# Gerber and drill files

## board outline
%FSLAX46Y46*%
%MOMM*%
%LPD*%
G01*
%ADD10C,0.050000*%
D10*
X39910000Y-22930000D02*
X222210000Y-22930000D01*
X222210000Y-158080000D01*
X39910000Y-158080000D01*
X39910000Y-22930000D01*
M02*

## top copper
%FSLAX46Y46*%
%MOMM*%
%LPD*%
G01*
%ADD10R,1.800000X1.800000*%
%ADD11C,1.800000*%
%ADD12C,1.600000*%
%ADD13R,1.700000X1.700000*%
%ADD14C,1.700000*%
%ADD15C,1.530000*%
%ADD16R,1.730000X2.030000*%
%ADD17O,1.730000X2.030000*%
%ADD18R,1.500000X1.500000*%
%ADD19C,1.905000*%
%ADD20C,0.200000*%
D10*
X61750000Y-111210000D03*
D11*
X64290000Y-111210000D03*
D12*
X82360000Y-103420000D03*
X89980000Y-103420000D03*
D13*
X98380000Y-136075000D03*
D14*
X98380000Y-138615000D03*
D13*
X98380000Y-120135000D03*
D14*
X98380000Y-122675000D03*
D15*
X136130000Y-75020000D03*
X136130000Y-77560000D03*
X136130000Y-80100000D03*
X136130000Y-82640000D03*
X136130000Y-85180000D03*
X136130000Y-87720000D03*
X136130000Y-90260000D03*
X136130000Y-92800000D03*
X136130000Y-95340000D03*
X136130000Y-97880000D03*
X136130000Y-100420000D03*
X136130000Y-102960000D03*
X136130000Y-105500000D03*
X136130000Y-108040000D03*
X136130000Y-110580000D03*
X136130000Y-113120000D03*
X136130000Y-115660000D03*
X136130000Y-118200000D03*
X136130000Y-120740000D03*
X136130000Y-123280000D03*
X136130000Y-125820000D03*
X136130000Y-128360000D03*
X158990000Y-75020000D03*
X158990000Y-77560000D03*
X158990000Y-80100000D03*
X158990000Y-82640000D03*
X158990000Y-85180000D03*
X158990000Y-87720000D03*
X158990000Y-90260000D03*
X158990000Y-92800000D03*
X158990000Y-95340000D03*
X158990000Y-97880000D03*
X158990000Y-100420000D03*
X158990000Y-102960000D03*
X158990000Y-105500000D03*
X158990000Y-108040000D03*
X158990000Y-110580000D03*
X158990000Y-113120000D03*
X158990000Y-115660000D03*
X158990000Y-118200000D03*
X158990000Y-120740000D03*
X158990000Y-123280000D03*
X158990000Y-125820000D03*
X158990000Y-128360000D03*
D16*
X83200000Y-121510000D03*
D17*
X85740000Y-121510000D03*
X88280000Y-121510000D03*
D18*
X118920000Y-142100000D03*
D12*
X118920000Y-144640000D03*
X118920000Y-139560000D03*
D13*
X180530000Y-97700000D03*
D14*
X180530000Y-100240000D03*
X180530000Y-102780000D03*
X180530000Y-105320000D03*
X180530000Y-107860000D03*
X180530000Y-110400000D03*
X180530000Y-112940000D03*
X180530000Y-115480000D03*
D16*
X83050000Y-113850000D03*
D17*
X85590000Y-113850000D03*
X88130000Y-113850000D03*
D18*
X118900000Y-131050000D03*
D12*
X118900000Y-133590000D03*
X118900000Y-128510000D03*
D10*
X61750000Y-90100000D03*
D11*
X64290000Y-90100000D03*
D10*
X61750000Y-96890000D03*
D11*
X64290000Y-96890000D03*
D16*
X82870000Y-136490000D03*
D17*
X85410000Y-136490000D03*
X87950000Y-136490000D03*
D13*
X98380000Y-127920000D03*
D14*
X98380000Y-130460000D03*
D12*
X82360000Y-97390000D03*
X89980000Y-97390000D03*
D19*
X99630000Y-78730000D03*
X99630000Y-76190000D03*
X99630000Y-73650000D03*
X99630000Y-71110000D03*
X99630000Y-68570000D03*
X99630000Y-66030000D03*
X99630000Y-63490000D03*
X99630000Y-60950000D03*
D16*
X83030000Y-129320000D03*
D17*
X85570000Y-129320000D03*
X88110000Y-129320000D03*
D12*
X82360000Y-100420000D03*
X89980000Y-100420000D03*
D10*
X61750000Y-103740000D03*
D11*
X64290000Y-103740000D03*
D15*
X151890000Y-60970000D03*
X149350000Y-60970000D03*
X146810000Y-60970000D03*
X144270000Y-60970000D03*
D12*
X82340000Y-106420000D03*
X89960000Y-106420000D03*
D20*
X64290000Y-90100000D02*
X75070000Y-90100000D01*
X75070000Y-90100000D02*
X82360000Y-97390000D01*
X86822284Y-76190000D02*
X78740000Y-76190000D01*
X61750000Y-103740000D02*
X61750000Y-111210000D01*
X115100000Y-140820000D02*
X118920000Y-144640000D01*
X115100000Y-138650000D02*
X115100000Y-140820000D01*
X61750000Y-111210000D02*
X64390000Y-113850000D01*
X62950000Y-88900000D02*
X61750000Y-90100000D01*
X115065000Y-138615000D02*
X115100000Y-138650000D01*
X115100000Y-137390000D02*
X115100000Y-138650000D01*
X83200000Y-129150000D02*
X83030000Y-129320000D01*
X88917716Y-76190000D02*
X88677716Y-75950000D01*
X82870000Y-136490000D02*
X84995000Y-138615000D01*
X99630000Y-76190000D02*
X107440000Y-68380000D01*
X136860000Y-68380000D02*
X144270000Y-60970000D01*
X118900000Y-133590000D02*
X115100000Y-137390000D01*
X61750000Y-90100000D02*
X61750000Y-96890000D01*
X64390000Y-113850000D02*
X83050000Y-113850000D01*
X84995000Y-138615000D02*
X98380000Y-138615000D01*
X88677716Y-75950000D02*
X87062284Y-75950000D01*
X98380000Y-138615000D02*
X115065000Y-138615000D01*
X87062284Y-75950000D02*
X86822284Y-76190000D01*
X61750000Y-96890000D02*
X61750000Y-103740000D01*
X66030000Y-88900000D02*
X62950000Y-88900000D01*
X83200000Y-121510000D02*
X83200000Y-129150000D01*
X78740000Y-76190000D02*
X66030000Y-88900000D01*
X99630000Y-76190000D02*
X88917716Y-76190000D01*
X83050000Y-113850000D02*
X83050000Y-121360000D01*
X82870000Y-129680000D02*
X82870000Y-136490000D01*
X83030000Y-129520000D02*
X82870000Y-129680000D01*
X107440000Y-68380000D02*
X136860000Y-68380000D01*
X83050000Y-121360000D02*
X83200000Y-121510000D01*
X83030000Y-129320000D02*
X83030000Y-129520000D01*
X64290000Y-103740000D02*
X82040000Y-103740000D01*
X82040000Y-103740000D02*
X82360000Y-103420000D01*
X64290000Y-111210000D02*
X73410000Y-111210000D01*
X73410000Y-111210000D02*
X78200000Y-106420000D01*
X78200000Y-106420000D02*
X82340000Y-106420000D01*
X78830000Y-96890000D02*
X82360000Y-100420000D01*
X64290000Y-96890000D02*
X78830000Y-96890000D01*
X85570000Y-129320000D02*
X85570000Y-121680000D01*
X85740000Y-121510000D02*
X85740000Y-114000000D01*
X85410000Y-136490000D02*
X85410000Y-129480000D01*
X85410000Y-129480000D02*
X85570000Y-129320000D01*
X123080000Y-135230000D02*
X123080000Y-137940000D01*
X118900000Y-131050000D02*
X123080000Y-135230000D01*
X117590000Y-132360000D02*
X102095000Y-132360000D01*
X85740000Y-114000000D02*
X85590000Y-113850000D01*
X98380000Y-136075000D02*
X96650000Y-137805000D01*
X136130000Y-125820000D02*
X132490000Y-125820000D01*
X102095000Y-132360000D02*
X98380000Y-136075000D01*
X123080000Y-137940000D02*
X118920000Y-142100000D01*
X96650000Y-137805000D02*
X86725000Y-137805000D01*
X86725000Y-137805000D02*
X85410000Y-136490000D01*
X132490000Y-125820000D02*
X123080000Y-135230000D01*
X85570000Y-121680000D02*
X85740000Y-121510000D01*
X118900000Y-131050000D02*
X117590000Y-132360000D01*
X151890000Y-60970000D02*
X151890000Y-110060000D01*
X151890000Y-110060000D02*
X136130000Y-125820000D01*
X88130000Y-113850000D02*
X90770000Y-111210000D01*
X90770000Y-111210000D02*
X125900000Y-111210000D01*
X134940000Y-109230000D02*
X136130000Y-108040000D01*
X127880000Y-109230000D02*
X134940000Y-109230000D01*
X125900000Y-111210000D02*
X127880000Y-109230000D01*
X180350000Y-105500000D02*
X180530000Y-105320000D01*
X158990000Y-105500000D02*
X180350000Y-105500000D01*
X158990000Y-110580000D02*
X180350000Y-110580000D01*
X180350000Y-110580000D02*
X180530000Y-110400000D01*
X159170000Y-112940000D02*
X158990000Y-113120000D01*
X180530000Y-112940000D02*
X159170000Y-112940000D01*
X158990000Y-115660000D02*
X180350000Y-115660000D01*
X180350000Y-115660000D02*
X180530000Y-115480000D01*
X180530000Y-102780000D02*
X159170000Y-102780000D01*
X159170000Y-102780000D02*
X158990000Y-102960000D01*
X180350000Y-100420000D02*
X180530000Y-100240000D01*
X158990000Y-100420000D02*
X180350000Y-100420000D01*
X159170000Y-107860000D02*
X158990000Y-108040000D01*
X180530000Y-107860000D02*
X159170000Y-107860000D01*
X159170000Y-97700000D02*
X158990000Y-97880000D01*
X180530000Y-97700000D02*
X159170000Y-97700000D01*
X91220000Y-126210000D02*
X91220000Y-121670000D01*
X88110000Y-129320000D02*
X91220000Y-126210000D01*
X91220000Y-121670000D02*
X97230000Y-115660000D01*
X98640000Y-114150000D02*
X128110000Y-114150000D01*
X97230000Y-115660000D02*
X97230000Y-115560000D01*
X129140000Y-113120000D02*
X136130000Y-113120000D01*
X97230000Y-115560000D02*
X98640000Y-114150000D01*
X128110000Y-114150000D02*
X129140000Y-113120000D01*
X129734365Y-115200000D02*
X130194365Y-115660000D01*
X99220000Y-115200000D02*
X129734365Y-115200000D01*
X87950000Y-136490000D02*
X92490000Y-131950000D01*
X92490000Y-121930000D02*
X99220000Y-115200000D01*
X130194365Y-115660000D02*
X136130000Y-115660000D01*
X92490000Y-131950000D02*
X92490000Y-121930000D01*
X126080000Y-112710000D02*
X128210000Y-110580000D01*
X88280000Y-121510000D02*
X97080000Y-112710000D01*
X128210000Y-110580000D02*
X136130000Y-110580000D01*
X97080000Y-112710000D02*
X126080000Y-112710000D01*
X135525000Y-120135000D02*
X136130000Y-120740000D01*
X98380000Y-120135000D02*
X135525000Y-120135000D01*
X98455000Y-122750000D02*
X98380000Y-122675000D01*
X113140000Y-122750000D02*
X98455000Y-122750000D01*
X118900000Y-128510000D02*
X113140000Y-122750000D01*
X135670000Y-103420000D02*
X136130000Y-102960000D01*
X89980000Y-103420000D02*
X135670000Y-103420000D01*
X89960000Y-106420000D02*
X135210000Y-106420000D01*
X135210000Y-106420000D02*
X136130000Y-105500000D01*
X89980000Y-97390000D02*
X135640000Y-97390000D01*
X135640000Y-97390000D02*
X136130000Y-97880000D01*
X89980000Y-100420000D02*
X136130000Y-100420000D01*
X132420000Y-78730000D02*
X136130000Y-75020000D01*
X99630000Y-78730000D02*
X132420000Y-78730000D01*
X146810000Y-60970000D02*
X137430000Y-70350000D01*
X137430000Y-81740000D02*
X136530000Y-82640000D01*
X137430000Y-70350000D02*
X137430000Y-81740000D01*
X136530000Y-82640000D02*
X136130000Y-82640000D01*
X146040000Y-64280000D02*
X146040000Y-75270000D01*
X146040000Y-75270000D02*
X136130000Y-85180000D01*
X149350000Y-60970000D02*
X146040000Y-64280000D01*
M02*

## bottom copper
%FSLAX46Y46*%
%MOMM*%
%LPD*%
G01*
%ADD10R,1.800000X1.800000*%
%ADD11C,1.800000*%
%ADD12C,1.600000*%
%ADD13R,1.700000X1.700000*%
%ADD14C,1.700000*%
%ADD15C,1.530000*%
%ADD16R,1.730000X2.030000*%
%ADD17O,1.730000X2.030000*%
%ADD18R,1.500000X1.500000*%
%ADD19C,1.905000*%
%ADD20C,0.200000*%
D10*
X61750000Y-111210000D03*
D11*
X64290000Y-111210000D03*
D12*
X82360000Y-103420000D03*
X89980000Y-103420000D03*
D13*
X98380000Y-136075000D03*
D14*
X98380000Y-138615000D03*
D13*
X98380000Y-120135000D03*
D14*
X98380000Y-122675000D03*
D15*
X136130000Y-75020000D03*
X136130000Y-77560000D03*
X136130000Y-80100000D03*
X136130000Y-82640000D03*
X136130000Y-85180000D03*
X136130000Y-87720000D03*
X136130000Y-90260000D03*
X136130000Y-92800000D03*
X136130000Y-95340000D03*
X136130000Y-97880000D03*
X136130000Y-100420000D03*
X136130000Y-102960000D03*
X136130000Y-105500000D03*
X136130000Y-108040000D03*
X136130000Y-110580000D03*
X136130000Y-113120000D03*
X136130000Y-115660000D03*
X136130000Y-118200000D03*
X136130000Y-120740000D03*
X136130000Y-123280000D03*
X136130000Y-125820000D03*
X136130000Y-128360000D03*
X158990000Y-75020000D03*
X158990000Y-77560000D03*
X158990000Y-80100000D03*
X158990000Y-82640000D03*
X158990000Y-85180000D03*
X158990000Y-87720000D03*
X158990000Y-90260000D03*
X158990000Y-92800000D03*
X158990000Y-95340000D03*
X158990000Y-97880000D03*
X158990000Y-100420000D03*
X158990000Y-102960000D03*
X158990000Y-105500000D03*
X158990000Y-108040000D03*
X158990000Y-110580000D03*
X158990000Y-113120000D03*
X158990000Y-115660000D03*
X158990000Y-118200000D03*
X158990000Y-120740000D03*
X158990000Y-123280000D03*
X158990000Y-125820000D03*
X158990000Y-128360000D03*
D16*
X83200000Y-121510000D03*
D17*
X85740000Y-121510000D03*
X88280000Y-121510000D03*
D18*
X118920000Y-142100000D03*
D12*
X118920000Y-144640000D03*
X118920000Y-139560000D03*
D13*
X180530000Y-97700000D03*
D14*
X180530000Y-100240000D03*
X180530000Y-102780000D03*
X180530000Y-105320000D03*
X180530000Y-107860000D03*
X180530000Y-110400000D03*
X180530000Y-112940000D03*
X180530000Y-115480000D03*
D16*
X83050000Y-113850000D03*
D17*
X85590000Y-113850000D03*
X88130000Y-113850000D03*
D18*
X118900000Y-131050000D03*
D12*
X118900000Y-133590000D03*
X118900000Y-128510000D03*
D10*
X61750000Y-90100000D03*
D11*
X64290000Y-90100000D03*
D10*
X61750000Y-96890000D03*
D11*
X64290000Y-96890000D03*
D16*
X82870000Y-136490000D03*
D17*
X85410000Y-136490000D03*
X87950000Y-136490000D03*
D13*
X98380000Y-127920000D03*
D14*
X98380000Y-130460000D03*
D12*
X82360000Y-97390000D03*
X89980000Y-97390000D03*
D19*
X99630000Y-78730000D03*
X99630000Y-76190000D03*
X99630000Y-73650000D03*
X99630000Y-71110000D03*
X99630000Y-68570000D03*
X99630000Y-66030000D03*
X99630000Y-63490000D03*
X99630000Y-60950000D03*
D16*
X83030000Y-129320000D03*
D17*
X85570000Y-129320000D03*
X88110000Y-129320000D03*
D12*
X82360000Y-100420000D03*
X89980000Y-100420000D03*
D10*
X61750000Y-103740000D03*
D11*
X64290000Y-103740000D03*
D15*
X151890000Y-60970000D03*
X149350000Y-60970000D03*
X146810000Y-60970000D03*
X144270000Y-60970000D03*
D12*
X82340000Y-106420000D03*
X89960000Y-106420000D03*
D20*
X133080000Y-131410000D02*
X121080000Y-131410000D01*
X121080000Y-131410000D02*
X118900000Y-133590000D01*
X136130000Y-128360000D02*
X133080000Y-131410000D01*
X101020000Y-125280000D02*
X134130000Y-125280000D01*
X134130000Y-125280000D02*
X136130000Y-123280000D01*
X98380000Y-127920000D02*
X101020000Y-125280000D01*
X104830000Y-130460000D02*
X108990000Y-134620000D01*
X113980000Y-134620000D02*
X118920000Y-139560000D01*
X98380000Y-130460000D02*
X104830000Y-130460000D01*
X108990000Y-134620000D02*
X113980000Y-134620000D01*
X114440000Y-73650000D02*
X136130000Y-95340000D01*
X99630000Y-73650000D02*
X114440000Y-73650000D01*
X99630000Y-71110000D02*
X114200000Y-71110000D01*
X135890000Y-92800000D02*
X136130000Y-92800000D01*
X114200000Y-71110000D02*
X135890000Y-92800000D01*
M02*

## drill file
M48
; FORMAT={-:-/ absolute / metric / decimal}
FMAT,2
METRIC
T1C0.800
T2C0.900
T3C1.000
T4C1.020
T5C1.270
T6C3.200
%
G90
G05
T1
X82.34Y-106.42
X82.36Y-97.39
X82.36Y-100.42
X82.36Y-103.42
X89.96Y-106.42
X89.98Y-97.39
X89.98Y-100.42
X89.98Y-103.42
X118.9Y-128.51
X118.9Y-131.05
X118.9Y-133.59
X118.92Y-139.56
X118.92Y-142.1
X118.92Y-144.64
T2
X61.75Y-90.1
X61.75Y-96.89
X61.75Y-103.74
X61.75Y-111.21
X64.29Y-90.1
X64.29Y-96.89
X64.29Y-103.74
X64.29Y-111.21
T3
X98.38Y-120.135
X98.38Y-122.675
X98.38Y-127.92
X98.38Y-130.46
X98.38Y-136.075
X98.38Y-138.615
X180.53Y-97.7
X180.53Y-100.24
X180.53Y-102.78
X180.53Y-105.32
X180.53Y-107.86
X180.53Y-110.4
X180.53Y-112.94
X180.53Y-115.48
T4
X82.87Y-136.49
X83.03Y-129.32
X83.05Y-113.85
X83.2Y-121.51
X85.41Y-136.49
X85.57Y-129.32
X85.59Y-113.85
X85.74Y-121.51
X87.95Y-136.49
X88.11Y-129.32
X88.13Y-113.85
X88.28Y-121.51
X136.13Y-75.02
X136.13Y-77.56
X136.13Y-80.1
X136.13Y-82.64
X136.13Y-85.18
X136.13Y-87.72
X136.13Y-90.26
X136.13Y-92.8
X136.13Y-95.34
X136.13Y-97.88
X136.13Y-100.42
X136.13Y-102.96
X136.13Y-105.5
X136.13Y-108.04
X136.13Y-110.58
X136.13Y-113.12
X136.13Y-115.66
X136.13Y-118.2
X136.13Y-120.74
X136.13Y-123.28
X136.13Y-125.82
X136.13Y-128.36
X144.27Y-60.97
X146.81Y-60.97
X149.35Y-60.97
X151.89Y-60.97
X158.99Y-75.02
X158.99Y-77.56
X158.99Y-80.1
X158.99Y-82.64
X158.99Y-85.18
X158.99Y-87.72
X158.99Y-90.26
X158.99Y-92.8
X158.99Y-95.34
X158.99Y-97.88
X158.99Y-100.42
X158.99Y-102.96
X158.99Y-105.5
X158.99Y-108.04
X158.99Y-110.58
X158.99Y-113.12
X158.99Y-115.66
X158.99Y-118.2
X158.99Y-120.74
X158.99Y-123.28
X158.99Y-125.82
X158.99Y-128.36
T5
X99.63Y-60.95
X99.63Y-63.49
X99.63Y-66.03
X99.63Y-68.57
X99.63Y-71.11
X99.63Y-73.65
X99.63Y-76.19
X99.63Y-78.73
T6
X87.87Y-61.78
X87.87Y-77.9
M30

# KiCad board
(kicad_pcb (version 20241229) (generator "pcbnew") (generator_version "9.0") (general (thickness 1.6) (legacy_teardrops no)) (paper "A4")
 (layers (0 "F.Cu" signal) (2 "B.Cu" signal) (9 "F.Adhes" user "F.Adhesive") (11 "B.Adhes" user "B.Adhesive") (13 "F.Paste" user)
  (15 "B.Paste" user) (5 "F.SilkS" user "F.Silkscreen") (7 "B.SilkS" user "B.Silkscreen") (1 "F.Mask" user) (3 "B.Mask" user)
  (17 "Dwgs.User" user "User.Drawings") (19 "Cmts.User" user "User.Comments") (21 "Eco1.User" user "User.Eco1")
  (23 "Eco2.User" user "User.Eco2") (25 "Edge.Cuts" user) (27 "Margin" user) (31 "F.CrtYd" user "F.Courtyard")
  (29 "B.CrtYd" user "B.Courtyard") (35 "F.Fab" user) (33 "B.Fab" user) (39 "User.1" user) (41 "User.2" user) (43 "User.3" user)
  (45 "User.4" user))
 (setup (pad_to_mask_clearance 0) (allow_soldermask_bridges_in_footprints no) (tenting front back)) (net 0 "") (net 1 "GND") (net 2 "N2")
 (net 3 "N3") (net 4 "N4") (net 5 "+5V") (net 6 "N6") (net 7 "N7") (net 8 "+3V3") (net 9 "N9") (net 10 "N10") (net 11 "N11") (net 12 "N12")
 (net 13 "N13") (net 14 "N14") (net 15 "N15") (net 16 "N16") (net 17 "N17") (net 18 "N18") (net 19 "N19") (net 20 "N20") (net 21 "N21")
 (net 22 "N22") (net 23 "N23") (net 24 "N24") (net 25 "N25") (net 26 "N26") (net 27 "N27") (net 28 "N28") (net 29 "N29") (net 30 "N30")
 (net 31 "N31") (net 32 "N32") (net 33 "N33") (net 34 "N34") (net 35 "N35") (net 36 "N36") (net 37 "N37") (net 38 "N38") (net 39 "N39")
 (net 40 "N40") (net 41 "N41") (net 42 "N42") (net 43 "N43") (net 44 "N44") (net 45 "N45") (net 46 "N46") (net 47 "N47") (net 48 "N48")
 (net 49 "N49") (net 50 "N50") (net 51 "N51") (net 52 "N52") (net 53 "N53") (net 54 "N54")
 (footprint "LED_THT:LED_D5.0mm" (layer "F.Cu") (at 61.75 111.21)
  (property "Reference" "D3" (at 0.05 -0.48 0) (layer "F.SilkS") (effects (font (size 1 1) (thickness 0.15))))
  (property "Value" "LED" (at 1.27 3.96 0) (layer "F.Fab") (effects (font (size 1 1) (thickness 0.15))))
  (pad "1" thru_hole rect (at 0 0) (size 1.8 1.8) (drill 0.9) (layers "*.Cu" "*.Mask") (remove_unused_layers no) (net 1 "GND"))
  (pad "2" thru_hole circle (at 2.54 0) (size 1.8 1.8) (drill 0.9) (layers "*.Cu" "*.Mask") (remove_unused_layers no) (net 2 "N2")))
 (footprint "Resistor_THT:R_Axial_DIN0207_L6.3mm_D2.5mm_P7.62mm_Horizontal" (layer "F.Cu") (at 82.36 103.42)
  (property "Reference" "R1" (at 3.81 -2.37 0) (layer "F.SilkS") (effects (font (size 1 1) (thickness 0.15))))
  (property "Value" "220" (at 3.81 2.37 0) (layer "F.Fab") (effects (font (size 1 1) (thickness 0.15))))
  (pad "1" thru_hole circle (at 0 0) (size 1.6 1.6) (drill 0.8) (layers "*.Cu" "*.Mask") (remove_unused_layers no) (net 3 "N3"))
  (pad "2" thru_hole circle (at 7.62 0) (size 1.6 1.6) (drill 0.8) (layers "*.Cu" "*.Mask") (remove_unused_layers no) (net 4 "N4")))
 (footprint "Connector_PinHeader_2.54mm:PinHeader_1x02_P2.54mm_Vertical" (layer "F.Cu") (at 98.38 136.075)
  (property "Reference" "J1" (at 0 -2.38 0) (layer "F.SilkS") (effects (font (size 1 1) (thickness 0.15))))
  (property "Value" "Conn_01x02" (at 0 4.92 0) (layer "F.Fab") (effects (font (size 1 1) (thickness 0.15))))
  (pad "1" thru_hole rect (at 0 0) (size 1.7 1.7) (drill 1) (layers "*.Cu" "*.Mask") (remove_unused_layers no) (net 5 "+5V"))
  (pad "2" thru_hole circle (at 0 2.54) (size 1.7 1.7) (drill 1) (layers "*.Cu" "*.Mask") (remove_unused_layers no) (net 1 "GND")))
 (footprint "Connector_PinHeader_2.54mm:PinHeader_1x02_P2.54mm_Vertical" (layer "F.Cu") (at 98.38 120.135)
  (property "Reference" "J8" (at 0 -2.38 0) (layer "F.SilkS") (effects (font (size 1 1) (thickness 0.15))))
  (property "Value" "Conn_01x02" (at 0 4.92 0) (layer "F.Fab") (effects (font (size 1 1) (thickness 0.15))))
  (pad "1" thru_hole rect (at 0 0) (size 1.7 1.7) (drill 1) (layers "*.Cu" "*.Mask") (remove_unused_layers no) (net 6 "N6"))
  (pad "2" thru_hole circle (at 0 2.54) (size 1.7 1.7) (drill 1) (layers "*.Cu" "*.Mask") (remove_unused_layers no) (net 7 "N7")))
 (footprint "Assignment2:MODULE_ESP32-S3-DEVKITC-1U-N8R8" (layer "F.Cu") (at 147.56 104.99)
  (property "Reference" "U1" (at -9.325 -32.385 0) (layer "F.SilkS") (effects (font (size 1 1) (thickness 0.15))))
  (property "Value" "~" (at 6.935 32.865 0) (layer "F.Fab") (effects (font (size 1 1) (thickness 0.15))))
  (pad "J1_1" thru_hole circle (at -11.43 -29.97) (size 1.53 1.53) (drill 1.02) (layers "*.Cu" "*.Mask") (remove_unused_layers no)
   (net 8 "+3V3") (solder_mask_margin 0.102))
  (pad "J1_2" thru_hole circle (at -11.43 -27.43) (size 1.53 1.53) (drill 1.02) (layers "*.Cu" "*.Mask") (remove_unused_layers no)
   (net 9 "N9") (solder_mask_margin 0.102))
  (pad "J1_3" thru_hole circle (at -11.43 -24.89) (size 1.53 1.53) (drill 1.02) (layers "*.Cu" "*.Mask") (remove_unused_layers no)
   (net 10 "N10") (solder_mask_margin 0.102))
  (pad "J1_4" thru_hole circle (at -11.43 -22.35) (size 1.53 1.53) (drill 1.02) (layers "*.Cu" "*.Mask") (remove_unused_layers no)
   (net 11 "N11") (solder_mask_margin 0.102))
  (pad "J1_5" thru_hole circle (at -11.43 -19.81) (size 1.53 1.53) (drill 1.02) (layers "*.Cu" "*.Mask") (remove_unused_layers no)
   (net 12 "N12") (solder_mask_margin 0.102))
  (pad "J1_6" thru_hole circle (at -11.43 -17.27) (size 1.53 1.53) (drill 1.02) (layers "*.Cu" "*.Mask") (remove_unused_layers no)
   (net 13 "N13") (solder_mask_margin 0.102))
  (pad "J1_7" thru_hole circle (at -11.43 -14.73) (size 1.53 1.53) (drill 1.02) (layers "*.Cu" "*.Mask") (remove_unused_layers no)
   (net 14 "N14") (solder_mask_margin 0.102))
  (pad "J1_8" thru_hole circle (at -11.43 -12.19) (size 1.53 1.53) (drill 1.02) (layers "*.Cu" "*.Mask") (remove_unused_layers no)
   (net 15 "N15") (solder_mask_margin 0.102))
  (pad "J1_9" thru_hole circle (at -11.43 -9.65) (size 1.53 1.53) (drill 1.02) (layers "*.Cu" "*.Mask") (remove_unused_layers no)
   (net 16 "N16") (solder_mask_margin 0.102))
  (pad "J1_10" thru_hole circle (at -11.43 -7.11) (size 1.53 1.53) (drill 1.02) (layers "*.Cu" "*.Mask") (remove_unused_layers no)
   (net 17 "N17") (solder_mask_margin 0.102))
  (pad "J1_11" thru_hole circle (at -11.43 -4.57) (size 1.53 1.53) (drill 1.02) (layers "*.Cu" "*.Mask") (remove_unused_layers no)
   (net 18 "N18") (solder_mask_margin 0.102))
  (pad "J1_12" thru_hole circle (at -11.43 -2.03) (size 1.53 1.53) (drill 1.02) (layers "*.Cu" "*.Mask") (remove_unused_layers no)
   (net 4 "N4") (solder_mask_margin 0.102))
  (pad "J1_13" thru_hole circle (at -11.43 0.51) (size 1.53 1.53) (drill 1.02) (layers "*.Cu" "*.Mask") (remove_unused_layers no)
   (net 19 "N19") (solder_mask_margin 0.102))
  (pad "J1_14" thru_hole circle (at -11.43 3.05) (size 1.53 1.53) (drill 1.02) (layers "*.Cu" "*.Mask") (remove_unused_layers no)
   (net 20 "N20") (solder_mask_margin 0.102))
  (pad "J1_15" thru_hole circle (at -11.43 5.59) (size 1.53 1.53) (drill 1.02) (layers "*.Cu" "*.Mask") (remove_unused_layers no)
   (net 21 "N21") (solder_mask_margin 0.102))
  (pad "J1_16" thru_hole circle (at -11.43 8.13) (size 1.53 1.53) (drill 1.02) (layers "*.Cu" "*.Mask") (remove_unused_layers no)
   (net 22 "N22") (solder_mask_margin 0.102))
  (pad "J1_17" thru_hole circle (at -11.43 10.67) (size 1.53 1.53) (drill 1.02) (layers "*.Cu" "*.Mask") (remove_unused_layers no)
   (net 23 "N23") (solder_mask_margin 0.102))
  (pad "J1_18" thru_hole circle (at -11.43 13.21) (size 1.53 1.53) (drill 1.02) (layers "*.Cu" "*.Mask") (remove_unused_layers no)
   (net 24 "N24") (solder_mask_margin 0.102))
  (pad "J1_19" thru_hole circle (at -11.43 15.75) (size 1.53 1.53) (drill 1.02) (layers "*.Cu" "*.Mask") (remove_unused_layers no)
   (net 6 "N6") (solder_mask_margin 0.102))
  (pad "J1_20" thru_hole circle (at -11.43 18.29) (size 1.53 1.53) (drill 1.02) (layers "*.Cu" "*.Mask") (remove_unused_layers no)
   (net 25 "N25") (solder_mask_margin 0.102))
  (pad "J1_21" thru_hole circle (at -11.43 20.83) (size 1.53 1.53) (drill 1.02) (layers "*.Cu" "*.Mask") (remove_unused_layers no)
   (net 5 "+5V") (solder_mask_margin 0.102))
  (pad "J1_22" thru_hole circle (at -11.43 23.37) (size 1.53 1.53) (drill 1.02) (layers "*.Cu" "*.Mask") (remove_unused_layers no)
   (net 1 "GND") (solder_mask_margin 0.102))
  (pad "J3_1" thru_hole circle (at 11.43 -29.97) (size 1.53 1.53) (drill 1.02) (layers "*.Cu" "*.Mask") (remove_unused_layers no)
   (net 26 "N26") (solder_mask_margin 0.102))
  (pad "J3_2" thru_hole circle (at 11.43 -27.43) (size 1.53 1.53) (drill 1.02) (layers "*.Cu" "*.Mask") (remove_unused_layers no)
   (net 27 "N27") (solder_mask_margin 0.102))
  (pad "J3_3" thru_hole circle (at 11.43 -24.89) (size 1.53 1.53) (drill 1.02) (layers "*.Cu" "*.Mask") (remove_unused_layers no)
   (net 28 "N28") (solder_mask_margin 0.102))
  (pad "J3_4" thru_hole circle (at 11.43 -22.35) (size 1.53 1.53) (drill 1.02) (layers "*.Cu" "*.Mask") (remove_unused_layers no)
   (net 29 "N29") (solder_mask_margin 0.102))
  (pad "J3_5" thru_hole circle (at 11.43 -19.81) (size 1.53 1.53) (drill 1.02) (layers "*.Cu" "*.Mask") (remove_unused_layers no)
   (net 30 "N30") (solder_mask_margin 0.102))
  (pad "J3_6" thru_hole circle (at 11.43 -17.27) (size 1.53 1.53) (drill 1.02) (layers "*.Cu" "*.Mask") (remove_unused_layers no)
   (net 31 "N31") (solder_mask_margin 0.102))
  (pad "J3_7" thru_hole circle (at 11.43 -14.73) (size 1.53 1.53) (drill 1.02) (layers "*.Cu" "*.Mask") (remove_unused_layers no)
   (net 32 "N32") (solder_mask_margin 0.102))
  (pad "J3_8" thru_hole circle (at 11.43 -12.19) (size 1.53 1.53) (drill 1.02) (layers "*.Cu" "*.Mask") (remove_unused_layers no)
   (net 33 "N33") (solder_mask_margin 0.102))
  (pad "J3_9" thru_hole circle (at 11.43 -9.65) (size 1.53 1.53) (drill 1.02) (layers "*.Cu" "*.Mask") (remove_unused_layers no)
   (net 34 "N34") (solder_mask_margin 0.102))
  (pad "J3_10" thru_hole circle (at 11.43 -7.11) (size 1.53 1.53) (drill 1.02) (layers "*.Cu" "*.Mask") (remove_unused_layers no)
   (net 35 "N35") (solder_mask_margin 0.102))
  (pad "J3_11" thru_hole circle (at 11.43 -4.57) (size 1.53 1.53) (drill 1.02) (layers "*.Cu" "*.Mask") (remove_unused_layers no)
   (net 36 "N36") (solder_mask_margin 0.102))
  (pad "J3_12" thru_hole circle (at 11.43 -2.03) (size 1.53 1.53) (drill 1.02) (layers "*.Cu" "*.Mask") (remove_unused_layers no)
   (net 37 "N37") (solder_mask_margin 0.102))
  (pad "J3_13" thru_hole circle (at 11.43 0.51) (size 1.53 1.53) (drill 1.02) (layers "*.Cu" "*.Mask") (remove_unused_layers no)
   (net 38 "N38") (solder_mask_margin 0.102))
  (pad "J3_14" thru_hole circle (at 11.43 3.05) (size 1.53 1.53) (drill 1.02) (layers "*.Cu" "*.Mask") (remove_unused_layers no)
   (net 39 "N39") (solder_mask_margin 0.102))
  (pad "J3_15" thru_hole circle (at 11.43 5.59) (size 1.53 1.53) (drill 1.02) (layers "*.Cu" "*.Mask") (remove_unused_layers no)
   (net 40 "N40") (solder_mask_margin 0.102))
  (pad "J3_16" thru_hole circle (at 11.43 8.13) (size 1.53 1.53) (drill 1.02) (layers "*.Cu" "*.Mask") (remove_unused_layers no)
   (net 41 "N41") (solder_mask_margin 0.102))
  (pad "J3_17" thru_hole circle (at 11.43 10.67) (size 1.53 1.53) (drill 1.02) (layers "*.Cu" "*.Mask") (remove_unused_layers no)
   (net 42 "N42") (solder_mask_margin 0.102))
  (pad "J3_18" thru_hole circle (at 11.43 13.21) (size 1.53 1.53) (drill 1.02) (layers "*.Cu" "*.Mask") (remove_unused_layers no)
   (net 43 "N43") (solder_mask_margin 0.102))
  (pad "J3_19" thru_hole circle (at 11.43 15.75) (size 1.53 1.53) (drill 1.02) (layers "*.Cu" "*.Mask") (remove_unused_layers no)
   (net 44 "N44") (solder_mask_margin 0.102))
  (pad "J3_20" thru_hole circle (at 11.43 18.29) (size 1.53 1.53) (drill 1.02) (layers "*.Cu" "*.Mask") (remove_unused_layers no)
   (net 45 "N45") (solder_mask_margin 0.102))
  (pad "J3_21" thru_hole circle (at 11.43 20.83) (size 1.53 1.53) (drill 1.02) (layers "*.Cu" "*.Mask") (remove_unused_layers no)
   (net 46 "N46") (solder_mask_margin 0.102))
  (pad "J3_22" thru_hole circle (at 11.43 23.37) (size 1.53 1.53) (drill 1.02) (layers "*.Cu" "*.Mask") (remove_unused_layers no)
   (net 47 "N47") (solder_mask_margin 0.102)))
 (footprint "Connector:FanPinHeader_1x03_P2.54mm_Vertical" (layer "F.Cu") (at 83.2 121.51)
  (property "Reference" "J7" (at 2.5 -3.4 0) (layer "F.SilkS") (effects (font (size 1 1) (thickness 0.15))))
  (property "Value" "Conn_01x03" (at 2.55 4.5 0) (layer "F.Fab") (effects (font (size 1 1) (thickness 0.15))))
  (pad "1" thru_hole rect (at 0 0 90) (size 2.03 1.73) (drill 1.02) (layers "*.Cu" "*.Mask") (remove_unused_layers no) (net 1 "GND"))
  (pad "2" thru_hole oval (at 2.54 0 90) (size 2.03 1.73) (drill 1.02) (layers "*.Cu" "*.Mask") (remove_unused_layers no) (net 5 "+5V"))
  (pad "3" thru_hole oval (at 5.08 0 90) (size 2.03 1.73) (drill 1.02) (layers "*.Cu" "*.Mask") (remove_unused_layers no) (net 21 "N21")))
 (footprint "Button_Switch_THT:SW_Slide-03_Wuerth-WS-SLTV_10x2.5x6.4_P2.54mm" (layer "F.Cu") (at 118.92 142.1 90)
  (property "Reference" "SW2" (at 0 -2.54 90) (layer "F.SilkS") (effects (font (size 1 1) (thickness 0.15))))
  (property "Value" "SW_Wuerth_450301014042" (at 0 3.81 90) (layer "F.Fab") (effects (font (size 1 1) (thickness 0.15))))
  (pad "1" thru_hole rect (at 0 0 90) (size 1.5 1.5) (drill 0.8) (layers "*.Cu" "*.Mask") (remove_unused_layers no) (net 5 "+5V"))
  (pad "2" thru_hole circle (at -2.54 0 90) (size 1.6 1.6) (drill 0.8) (layers "*.Cu" "*.Mask") (remove_unused_layers no) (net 1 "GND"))
  (pad "3" thru_hole circle (at 2.54 0 90) (size 1.6 1.6) (drill 0.8) (layers "*.Cu" "*.Mask") (remove_unused_layers no) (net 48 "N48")))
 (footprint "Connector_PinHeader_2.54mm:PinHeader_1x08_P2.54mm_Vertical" (layer "F.Cu") (at 180.53 97.7)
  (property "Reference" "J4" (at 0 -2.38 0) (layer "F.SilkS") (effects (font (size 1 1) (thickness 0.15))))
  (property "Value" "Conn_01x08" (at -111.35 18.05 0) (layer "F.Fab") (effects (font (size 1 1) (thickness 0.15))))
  (pad "1" thru_hole rect (at 0 0) (size 1.7 1.7) (drill 1) (layers "*.Cu" "*.Mask") (remove_unused_layers no) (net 35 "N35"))
  (pad "2" thru_hole circle (at 0 2.54) (size 1.7 1.7) (drill 1) (layers "*.Cu" "*.Mask") (remove_unused_layers no) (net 36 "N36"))
  (pad "3" thru_hole circle (at 0 5.08) (size 1.7 1.7) (drill 1) (layers "*.Cu" "*.Mask") (remove_unused_layers no) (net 37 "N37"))
  (pad "4" thru_hole circle (at 0 7.62) (size 1.7 1.7) (drill 1) (layers "*.Cu" "*.Mask") (remove_unused_layers no) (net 38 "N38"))
  (pad "5" thru_hole circle (at 0 10.16) (size 1.7 1.7) (drill 1) (layers "*.Cu" "*.Mask") (remove_unused_layers no) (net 39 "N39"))
  (pad "6" thru_hole circle (at 0 12.7) (size 1.7 1.7) (drill 1) (layers "*.Cu" "*.Mask") (remove_unused_layers no) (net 40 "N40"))
  (pad "7" thru_hole circle (at 0 15.24) (size 1.7 1.7) (drill 1) (layers "*.Cu" "*.Mask") (remove_unused_layers no) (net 41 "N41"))
  (pad "8" thru_hole circle (at 0 17.78) (size 1.7 1.7) (drill 1) (layers "*.Cu" "*.Mask") (remove_unused_layers no) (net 42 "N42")))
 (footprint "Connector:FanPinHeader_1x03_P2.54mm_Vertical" (layer "F.Cu") (at 83.05 113.85)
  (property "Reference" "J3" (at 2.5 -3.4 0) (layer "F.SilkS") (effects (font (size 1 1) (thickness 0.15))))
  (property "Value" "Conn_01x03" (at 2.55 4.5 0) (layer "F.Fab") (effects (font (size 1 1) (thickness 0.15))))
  (pad "1" thru_hole rect (at 0 0 90) (size 2.03 1.73) (drill 1.02) (layers "*.Cu" "*.Mask") (remove_unused_layers no) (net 1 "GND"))
  (pad "2" thru_hole oval (at 2.54 0 90) (size 2.03 1.73) (drill 1.02) (layers "*.Cu" "*.Mask") (remove_unused_layers no) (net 5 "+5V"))
  (pad "3" thru_hole oval (at 5.08 0 90) (size 2.03 1.73) (drill 1.02) (layers "*.Cu" "*.Mask") (remove_unused_layers no) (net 20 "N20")))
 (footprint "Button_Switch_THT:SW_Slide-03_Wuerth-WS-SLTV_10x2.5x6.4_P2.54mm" (layer "F.Cu") (at 118.9 131.05 90)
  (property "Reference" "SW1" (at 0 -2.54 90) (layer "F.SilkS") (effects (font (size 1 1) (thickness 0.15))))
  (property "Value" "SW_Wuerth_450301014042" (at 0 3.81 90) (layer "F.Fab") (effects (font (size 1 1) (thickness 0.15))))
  (pad "1" thru_hole rect (at 0 0 90) (size 1.5 1.5) (drill 0.8) (layers "*.Cu" "*.Mask") (remove_unused_layers no) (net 5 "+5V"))
  (pad "2" thru_hole circle (at -2.54 0 90) (size 1.6 1.6) (drill 0.8) (layers "*.Cu" "*.Mask") (remove_unused_layers no) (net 1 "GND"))
  (pad "3" thru_hole circle (at 2.54 0 90) (size 1.6 1.6) (drill 0.8) (layers "*.Cu" "*.Mask") (remove_unused_layers no) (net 7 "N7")))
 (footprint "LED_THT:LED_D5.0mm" (layer "F.Cu") (at 61.75 90.1)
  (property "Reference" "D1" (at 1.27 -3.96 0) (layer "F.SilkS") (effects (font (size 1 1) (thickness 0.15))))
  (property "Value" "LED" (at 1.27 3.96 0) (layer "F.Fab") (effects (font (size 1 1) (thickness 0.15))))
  (pad "1" thru_hole rect (at 0 0) (size 1.8 1.8) (drill 0.9) (layers "*.Cu" "*.Mask") (remove_unused_layers no) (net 1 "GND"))
  (pad "2" thru_hole circle (at 2.54 0) (size 1.8 1.8) (drill 0.9) (layers "*.Cu" "*.Mask") (remove_unused_layers no) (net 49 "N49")))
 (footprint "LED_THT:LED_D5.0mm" (layer "F.Cu") (at 61.75 96.89)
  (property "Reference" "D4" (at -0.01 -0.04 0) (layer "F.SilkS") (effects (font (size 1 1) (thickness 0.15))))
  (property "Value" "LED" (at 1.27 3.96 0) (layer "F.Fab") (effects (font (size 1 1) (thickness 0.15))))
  (pad "1" thru_hole rect (at 0 0) (size 1.8 1.8) (drill 0.9) (layers "*.Cu" "*.Mask") (remove_unused_layers no) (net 1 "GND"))
  (pad "2" thru_hole circle (at 2.54 0) (size 1.8 1.8) (drill 0.9) (layers "*.Cu" "*.Mask") (remove_unused_layers no) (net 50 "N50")))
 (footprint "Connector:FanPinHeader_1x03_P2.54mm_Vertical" (layer "F.Cu") (at 82.87 136.49)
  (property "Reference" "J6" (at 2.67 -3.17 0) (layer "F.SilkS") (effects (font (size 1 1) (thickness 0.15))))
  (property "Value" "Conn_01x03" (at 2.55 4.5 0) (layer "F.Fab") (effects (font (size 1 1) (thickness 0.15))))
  (pad "1" thru_hole rect (at 0 0 90) (size 2.03 1.73) (drill 1.02) (layers "*.Cu" "*.Mask") (remove_unused_layers no) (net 1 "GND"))
  (pad "2" thru_hole oval (at 2.54 0 90) (size 2.03 1.73) (drill 1.02) (layers "*.Cu" "*.Mask") (remove_unused_layers no) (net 5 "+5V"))
  (pad "3" thru_hole oval (at 5.08 0 90) (size 2.03 1.73) (drill 1.02) (layers "*.Cu" "*.Mask") (remove_unused_layers no) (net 23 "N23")))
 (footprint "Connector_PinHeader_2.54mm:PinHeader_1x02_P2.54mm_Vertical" (layer "F.Cu") (at 98.38 127.92)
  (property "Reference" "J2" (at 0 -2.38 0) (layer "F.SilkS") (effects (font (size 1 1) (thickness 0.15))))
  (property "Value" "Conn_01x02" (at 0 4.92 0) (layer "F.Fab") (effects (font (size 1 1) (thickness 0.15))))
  (pad "1" thru_hole rect (at 0 0) (size 1.7 1.7) (drill 1) (layers "*.Cu" "*.Mask") (remove_unused_layers no) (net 25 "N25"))
  (pad "2" thru_hole circle (at 0 2.54) (size 1.7 1.7) (drill 1) (layers "*.Cu" "*.Mask") (remove_unused_layers no) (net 48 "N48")))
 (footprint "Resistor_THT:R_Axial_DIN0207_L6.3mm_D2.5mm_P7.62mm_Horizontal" (layer "F.Cu") (at 82.36 97.39)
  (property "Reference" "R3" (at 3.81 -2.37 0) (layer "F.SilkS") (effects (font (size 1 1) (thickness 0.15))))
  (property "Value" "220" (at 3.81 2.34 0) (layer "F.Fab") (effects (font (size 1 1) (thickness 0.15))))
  (pad "1" thru_hole circle (at 0 0) (size 1.6 1.6) (drill 0.8) (layers "*.Cu" "*.Mask") (remove_unused_layers no) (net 49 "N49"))
  (pad "2" thru_hole circle (at 7.62 0) (size 1.6 1.6) (drill 0.8) (layers "*.Cu" "*.Mask") (remove_unused_layers no) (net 17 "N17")))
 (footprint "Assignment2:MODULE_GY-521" (layer "F.Cu") (at 93.3 69.84 180)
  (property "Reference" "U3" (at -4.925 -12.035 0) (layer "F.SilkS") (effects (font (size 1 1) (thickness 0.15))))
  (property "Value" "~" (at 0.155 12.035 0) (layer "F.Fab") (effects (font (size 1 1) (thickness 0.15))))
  (pad "" np_thru_hole circle (at 5.43 -8.06 180) (size 3.2 3.2) (drill 3.2) (layers "*.Cu" "*.Mask"))
  (pad "" np_thru_hole circle (at 5.43 8.06 180) (size 3.2 3.2) (drill 3.2) (layers "*.Cu" "*.Mask"))
  (pad "1" thru_hole circle (at -6.33 -8.89 180) (size 1.905 1.905) (drill 1.27) (layers "*.Cu" "*.Mask") (remove_unused_layers no)
   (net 8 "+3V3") (solder_mask_margin 0.102))
  (pad "2" thru_hole circle (at -6.33 -6.35 180) (size 1.905 1.905) (drill 1.27) (layers "*.Cu" "*.Mask") (remove_unused_layers no)
   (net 1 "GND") (solder_mask_margin 0.102))
  (pad "3" thru_hole circle (at -6.33 -3.81 180) (size 1.905 1.905) (drill 1.27) (layers "*.Cu" "*.Mask") (remove_unused_layers no)
   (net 16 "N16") (solder_mask_margin 0.102))
  (pad "4" thru_hole circle (at -6.33 -1.27 180) (size 1.905 1.905) (drill 1.27) (layers "*.Cu" "*.Mask") (remove_unused_layers no)
   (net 15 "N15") (solder_mask_margin 0.102))
  (pad "5" thru_hole circle (at -6.33 1.27 180) (size 1.905 1.905) (drill 1.27) (layers "*.Cu" "*.Mask") (remove_unused_layers no)
   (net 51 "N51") (solder_mask_margin 0.102))
  (pad "6" thru_hole circle (at -6.33 3.81 180) (size 1.905 1.905) (drill 1.27) (layers "*.Cu" "*.Mask") (remove_unused_layers no)
   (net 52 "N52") (solder_mask_margin 0.102))
  (pad "7" thru_hole circle (at -6.33 6.35 180) (size 1.905 1.905) (drill 1.27) (layers "*.Cu" "*.Mask") (remove_unused_layers no)
   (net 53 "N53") (solder_mask_margin 0.102))
  (pad "8" thru_hole circle (at -6.33 8.89 180) (size 1.905 1.905) (drill 1.27) (layers "*.Cu" "*.Mask") (remove_unused_layers no)
   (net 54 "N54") (solder_mask_margin 0.102)))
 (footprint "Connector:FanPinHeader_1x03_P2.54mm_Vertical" (layer "F.Cu") (at 83.03 129.32)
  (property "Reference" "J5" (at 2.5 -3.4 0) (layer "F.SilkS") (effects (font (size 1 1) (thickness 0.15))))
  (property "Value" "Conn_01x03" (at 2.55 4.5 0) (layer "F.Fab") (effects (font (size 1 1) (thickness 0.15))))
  (pad "1" thru_hole rect (at 0 0 90) (size 2.03 1.73) (drill 1.02) (layers "*.Cu" "*.Mask") (remove_unused_layers no) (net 1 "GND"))
  (pad "2" thru_hole oval (at 2.54 0 90) (size 2.03 1.73) (drill 1.02) (layers "*.Cu" "*.Mask") (remove_unused_layers no) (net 5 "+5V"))
  (pad "3" thru_hole oval (at 5.08 0 90) (size 2.03 1.73) (drill 1.02) (layers "*.Cu" "*.Mask") (remove_unused_layers no) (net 22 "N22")))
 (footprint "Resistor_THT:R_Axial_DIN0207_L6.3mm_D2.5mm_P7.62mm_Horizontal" (layer "F.Cu") (at 82.36 100.42)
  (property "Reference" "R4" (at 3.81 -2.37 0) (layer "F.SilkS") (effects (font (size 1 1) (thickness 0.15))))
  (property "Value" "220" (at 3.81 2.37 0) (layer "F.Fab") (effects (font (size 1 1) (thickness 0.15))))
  (pad "1" thru_hole circle (at 0 0) (size 1.6 1.6) (drill 0.8) (layers "*.Cu" "*.Mask") (remove_unused_layers no) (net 50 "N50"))
  (pad "2" thru_hole circle (at 7.62 0) (size 1.6 1.6) (drill 0.8) (layers "*.Cu" "*.Mask") (remove_unused_layers no) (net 18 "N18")))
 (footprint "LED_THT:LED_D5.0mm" (layer "F.Cu") (at 61.75 103.74)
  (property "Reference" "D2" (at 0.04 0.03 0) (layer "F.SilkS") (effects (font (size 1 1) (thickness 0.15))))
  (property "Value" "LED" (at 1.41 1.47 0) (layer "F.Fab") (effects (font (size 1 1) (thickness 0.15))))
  (pad "1" thru_hole rect (at 0 0) (size 1.8 1.8) (drill 0.9) (layers "*.Cu" "*.Mask") (remove_unused_layers no) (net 1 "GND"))
  (pad "2" thru_hole circle (at 2.54 0) (size 1.8 1.8) (drill 0.9) (layers "*.Cu" "*.Mask") (remove_unused_layers no) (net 3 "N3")))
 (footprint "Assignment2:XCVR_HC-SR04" (layer "F.Cu") (at 148.08 60.97 180)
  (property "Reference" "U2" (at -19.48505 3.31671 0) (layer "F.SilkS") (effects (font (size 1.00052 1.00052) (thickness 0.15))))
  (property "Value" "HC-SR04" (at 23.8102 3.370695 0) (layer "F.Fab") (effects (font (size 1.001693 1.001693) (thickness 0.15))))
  (pad "1" thru_hole circle (at -3.81 0 180) (size 1.53 1.53) (drill 1.02) (layers "*.Cu" "*.Mask") (remove_unused_layers no) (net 5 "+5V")
   (solder_mask_margin 0.102))
  (pad "2" thru_hole circle (at -1.27 0 180) (size 1.53 1.53) (drill 1.02) (layers "*.Cu" "*.Mask") (remove_unused_layers no) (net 12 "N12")
   (solder_mask_margin 0.102))
  (pad "3" thru_hole circle (at 1.27 0 180) (size 1.53 1.53) (drill 1.02) (layers "*.Cu" "*.Mask") (remove_unused_layers no) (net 11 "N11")
   (solder_mask_margin 0.102))
  (pad "4" thru_hole circle (at 3.81 0 180) (size 1.53 1.53) (drill 1.02) (layers "*.Cu" "*.Mask") (remove_unused_layers no) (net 1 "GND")
   (solder_mask_margin 0.102)))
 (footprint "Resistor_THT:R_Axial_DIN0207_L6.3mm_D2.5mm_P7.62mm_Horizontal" (layer "F.Cu") (at 82.34 106.42)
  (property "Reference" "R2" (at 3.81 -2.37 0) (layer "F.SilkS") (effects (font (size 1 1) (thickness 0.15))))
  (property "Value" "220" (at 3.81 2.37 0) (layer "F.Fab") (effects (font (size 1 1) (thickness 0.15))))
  (pad "1" thru_hole circle (at 0 0) (size 1.6 1.6) (drill 0.8) (layers "*.Cu" "*.Mask") (remove_unused_layers no) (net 2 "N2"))
  (pad "2" thru_hole circle (at 7.62 0) (size 1.6 1.6) (drill 0.8) (layers "*.Cu" "*.Mask") (remove_unused_layers no) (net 19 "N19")))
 (gr_rect (start 39.91 22.93) (end 222.21 158.08) (stroke (width 0.05) (type default)) (fill no) (layer "Edge.Cuts"))
 (segment (start 64.29 90.1) (end 75.07 90.1) (width 0.2) (layer "F.Cu") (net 49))
 (segment (start 75.07 90.1) (end 82.36 97.39) (width 0.2) (layer "F.Cu") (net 49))
 (segment (start 86.822284 76.19) (end 78.74 76.19) (width 0.2) (layer "F.Cu") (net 1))
 (segment (start 61.75 103.74) (end 61.75 111.21) (width 0.2) (layer "F.Cu") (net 1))
 (segment (start 115.1 140.82) (end 118.92 144.64) (width 0.2) (layer "F.Cu") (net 1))
 (segment (start 115.1 138.65) (end 115.1 140.82) (width 0.2) (layer "F.Cu") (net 1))
 (segment (start 61.75 111.21) (end 64.39 113.85) (width 0.2) (layer "F.Cu") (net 1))
 (segment (start 62.95 88.9) (end 61.75 90.1) (width 0.2) (layer "F.Cu") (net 1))
 (segment (start 115.065 138.615) (end 115.1 138.65) (width 0.2) (layer "F.Cu") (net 1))
 (segment (start 115.1 137.39) (end 115.1 138.65) (width 0.2) (layer "F.Cu") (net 1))
 (segment (start 83.2 129.15) (end 83.03 129.32) (width 0.2) (layer "F.Cu") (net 1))
 (segment (start 88.917716 76.19) (end 88.677716 75.95) (width 0.2) (layer "F.Cu") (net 1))
 (segment (start 82.87 136.49) (end 84.995 138.615) (width 0.2) (layer "F.Cu") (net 1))
 (segment (start 99.63 76.19) (end 107.44 68.38) (width 0.2) (layer "F.Cu") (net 1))
 (segment (start 136.86 68.38) (end 144.27 60.97) (width 0.2) (layer "F.Cu") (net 1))
 (segment (start 118.9 133.59) (end 115.1 137.39) (width 0.2) (layer "F.Cu") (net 1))
 (segment (start 61.75 90.1) (end 61.75 96.89) (width 0.2) (layer "F.Cu") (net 1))
 (segment (start 64.39 113.85) (end 83.05 113.85) (width 0.2) (layer "F.Cu") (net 1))
 (segment (start 84.995 138.615) (end 98.38 138.615) (width 0.2) (layer "F.Cu") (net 1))
 (segment (start 88.677716 75.95) (end 87.062284 75.95) (width 0.2) (layer "F.Cu") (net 1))
 (segment (start 98.38 138.615) (end 115.065 138.615) (width 0.2) (layer "F.Cu") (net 1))
 (segment (start 87.062284 75.95) (end 86.822284 76.19) (width 0.2) (layer "F.Cu") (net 1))
 (segment (start 61.75 96.89) (end 61.75 103.74) (width 0.2) (layer "F.Cu") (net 1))
 (segment (start 66.03 88.9) (end 62.95 88.9) (width 0.2) (layer "F.Cu") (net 1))
 (segment (start 83.2 121.51) (end 83.2 129.15) (width 0.2) (layer "F.Cu") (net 1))
 (segment (start 78.74 76.19) (end 66.03 88.9) (width 0.2) (layer "F.Cu") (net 1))
 (segment (start 99.63 76.19) (end 88.917716 76.19) (width 0.2) (layer "F.Cu") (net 1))
 (segment (start 83.05 113.85) (end 83.05 121.36) (width 0.2) (layer "F.Cu") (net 1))
 (segment (start 82.87 129.68) (end 82.87 136.49) (width 0.2) (layer "F.Cu") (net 1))
 (segment (start 83.03 129.52) (end 82.87 129.68) (width 0.2) (layer "F.Cu") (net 1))
 (segment (start 107.44 68.38) (end 136.86 68.38) (width 0.2) (layer "F.Cu") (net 1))
 (segment (start 83.05 121.36) (end 83.2 121.51) (width 0.2) (layer "F.Cu") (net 1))
 (segment (start 83.03 129.32) (end 83.03 129.52) (width 0.2) (layer "F.Cu") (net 1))
 (segment (start 133.08 131.41) (end 121.08 131.41) (width 0.2) (layer "B.Cu") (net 1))
 (segment (start 121.08 131.41) (end 118.9 133.59) (width 0.2) (layer "B.Cu") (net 1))
 (segment (start 136.13 128.36) (end 133.08 131.41) (width 0.2) (layer "B.Cu") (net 1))
 (segment (start 64.29 103.74) (end 82.04 103.74) (width 0.2) (layer "F.Cu") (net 3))
 (segment (start 82.04 103.74) (end 82.36 103.42) (width 0.2) (layer "F.Cu") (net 3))
 (segment (start 64.29 111.21) (end 73.41 111.21) (width 0.2) (layer "F.Cu") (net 2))
 (segment (start 73.41 111.21) (end 78.2 106.42) (width 0.2) (layer "F.Cu") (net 2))
 (segment (start 78.2 106.42) (end 82.34 106.42) (width 0.2) (layer "F.Cu") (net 2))
 (segment (start 78.83 96.89) (end 82.36 100.42) (width 0.2) (layer "F.Cu") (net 50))
 (segment (start 64.29 96.89) (end 78.83 96.89) (width 0.2) (layer "F.Cu") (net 50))
 (segment (start 85.57 129.32) (end 85.57 121.68) (width 0.2) (layer "F.Cu") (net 5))
 (segment (start 85.74 121.51) (end 85.74 114) (width 0.2) (layer "F.Cu") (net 5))
 (segment (start 85.41 136.49) (end 85.41 129.48) (width 0.2) (layer "F.Cu") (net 5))
 (segment (start 85.41 129.48) (end 85.57 129.32) (width 0.2) (layer "F.Cu") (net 5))
 (segment (start 123.08 135.23) (end 123.08 137.94) (width 0.2) (layer "F.Cu") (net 5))
 (segment (start 118.9 131.05) (end 123.08 135.23) (width 0.2) (layer "F.Cu") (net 5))
 (segment (start 117.59 132.36) (end 102.095 132.36) (width 0.2) (layer "F.Cu") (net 5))
 (segment (start 85.74 114) (end 85.59 113.85) (width 0.2) (layer "F.Cu") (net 5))
 (segment (start 98.38 136.075) (end 96.65 137.805) (width 0.2) (layer "F.Cu") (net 5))
 (segment (start 136.13 125.82) (end 132.49 125.82) (width 0.2) (layer "F.Cu") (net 5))
 (segment (start 102.095 132.36) (end 98.38 136.075) (width 0.2) (layer "F.Cu") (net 5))
 (segment (start 123.08 137.94) (end 118.92 142.1) (width 0.2) (layer "F.Cu") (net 5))
 (segment (start 96.65 137.805) (end 86.725 137.805) (width 0.2) (layer "F.Cu") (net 5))
 (segment (start 86.725 137.805) (end 85.41 136.49) (width 0.2) (layer "F.Cu") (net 5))
 (segment (start 132.49 125.82) (end 123.08 135.23) (width 0.2) (layer "F.Cu") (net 5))
 (segment (start 85.57 121.68) (end 85.74 121.51) (width 0.2) (layer "F.Cu") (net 5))
 (segment (start 118.9 131.05) (end 117.59 132.36) (width 0.2) (layer "F.Cu") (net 5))
 (segment (start 151.89 60.97) (end 151.89 110.06) (width 0.2) (layer "F.Cu") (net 5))
 (segment (start 151.89 110.06) (end 136.13 125.82) (width 0.2) (layer "F.Cu") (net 5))
 (segment (start 101.02 125.28) (end 134.13 125.28) (width 0.2) (layer "B.Cu") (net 25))
 (segment (start 134.13 125.28) (end 136.13 123.28) (width 0.2) (layer "B.Cu") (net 25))
 (segment (start 98.38 127.92) (end 101.02 125.28) (width 0.2) (layer "B.Cu") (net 25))
 (segment (start 104.83 130.46) (end 108.99 134.62) (width 0.2) (layer "B.Cu") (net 48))
 (segment (start 113.98 134.62) (end 118.92 139.56) (width 0.2) (layer "B.Cu") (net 48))
 (segment (start 98.38 130.46) (end 104.83 130.46) (width 0.2) (layer "B.Cu") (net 48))
 (segment (start 108.99 134.62) (end 113.98 134.62) (width 0.2) (layer "B.Cu") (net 48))
 (segment (start 88.13 113.85) (end 90.77 111.21) (width 0.2) (layer "F.Cu") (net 20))
 (segment (start 90.77 111.21) (end 125.9 111.21) (width 0.2) (layer "F.Cu") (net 20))
 (segment (start 134.94 109.23) (end 136.13 108.04) (width 0.2) (layer "F.Cu") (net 20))
 (segment (start 127.88 109.23) (end 134.94 109.23) (width 0.2) (layer "F.Cu") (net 20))
 (segment (start 125.9 111.21) (end 127.88 109.23) (width 0.2) (layer "F.Cu") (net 20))
 (segment (start 180.35 105.5) (end 180.53 105.32) (width 0.2) (layer "F.Cu") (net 38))
 (segment (start 158.99 105.5) (end 180.35 105.5) (width 0.2) (layer "F.Cu") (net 38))
 (segment (start 158.99 110.58) (end 180.35 110.58) (width 0.2) (layer "F.Cu") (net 40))
 (segment (start 180.35 110.58) (end 180.53 110.4) (width 0.2) (layer "F.Cu") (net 40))
 (segment (start 159.17 112.94) (end 158.99 113.12) (width 0.2) (layer "F.Cu") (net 41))
 (segment (start 180.53 112.94) (end 159.17 112.94) (width 0.2) (layer "F.Cu") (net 41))
 (segment (start 158.99 115.66) (end 180.35 115.66) (width 0.2) (layer "F.Cu") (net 42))
 (segment (start 180.35 115.66) (end 180.53 115.48) (width 0.2) (layer "F.Cu") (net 42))
 (segment (start 180.53 102.78) (end 159.17 102.78) (width 0.2) (layer "F.Cu") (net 37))
 (segment (start 159.17 102.78) (end 158.99 102.96) (width 0.2) (layer "F.Cu") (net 37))
 (segment (start 180.35 100.42) (end 180.53 100.24) (width 0.2) (layer "F.Cu") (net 36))
 (segment (start 158.99 100.42) (end 180.35 100.42) (width 0.2) (layer "F.Cu") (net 36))
 (segment (start 159.17 107.86) (end 158.99 108.04) (width 0.2) (layer "F.Cu") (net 39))
 (segment (start 180.53 107.86) (end 159.17 107.86) (width 0.2) (layer "F.Cu") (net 39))
 (segment (start 159.17 97.7) (end 158.99 97.88) (width 0.2) (layer "F.Cu") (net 35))
 (segment (start 180.53 97.7) (end 159.17 97.7) (width 0.2) (layer "F.Cu") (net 35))
 (segment (start 91.22 126.21) (end 91.22 121.67) (width 0.2) (layer "F.Cu") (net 22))
 (segment (start 88.11 129.32) (end 91.22 126.21) (width 0.2) (layer "F.Cu") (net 22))
 (segment (start 91.22 121.67) (end 97.23 115.66) (width 0.2) (layer "F.Cu") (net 22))
 (segment (start 98.64 114.15) (end 128.11 114.15) (width 0.2) (layer "F.Cu") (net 22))
 (segment (start 97.23 115.66) (end 97.23 115.56) (width 0.2) (layer "F.Cu") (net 22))
 (segment (start 129.14 113.12) (end 136.13 113.12) (width 0.2) (layer "F.Cu") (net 22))
 (segment (start 97.23 115.56) (end 98.64 114.15) (width 0.2) (layer "F.Cu") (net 22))
 (segment (start 128.11 114.15) (end 129.14 113.12) (width 0.2) (layer "F.Cu") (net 22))
 (segment (start 129.734365 115.2) (end 130.194365 115.66) (width 0.2) (layer "F.Cu") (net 23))
 (segment (start 99.22 115.2) (end 129.734365 115.2) (width 0.2) (layer "F.Cu") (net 23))
 (segment (start 87.95 136.49) (end 92.49 131.95) (width 0.2) (layer "F.Cu") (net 23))
 (segment (start 92.49 121.93) (end 99.22 115.2) (width 0.2) (layer "F.Cu") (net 23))
 (segment (start 130.194365 115.66) (end 136.13 115.66) (width 0.2) (layer "F.Cu") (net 23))
 (segment (start 92.49 131.95) (end 92.49 121.93) (width 0.2) (layer "F.Cu") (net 23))
 (segment (start 126.08 112.71) (end 128.21 110.58) (width 0.2) (layer "F.Cu") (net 21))
 (segment (start 88.28 121.51) (end 97.08 112.71) (width 0.2) (layer "F.Cu") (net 21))
 (segment (start 128.21 110.58) (end 136.13 110.58) (width 0.2) (layer "F.Cu") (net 21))
 (segment (start 97.08 112.71) (end 126.08 112.71) (width 0.2) (layer "F.Cu") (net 21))
 (segment (start 135.525 120.135) (end 136.13 120.74) (width 0.2) (layer "F.Cu") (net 6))
 (segment (start 98.38 120.135) (end 135.525 120.135) (width 0.2) (layer "F.Cu") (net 6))
 (segment (start 98.455 122.75) (end 98.38 122.675) (width 0.2) (layer "F.Cu") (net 7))
 (segment (start 113.14 122.75) (end 98.455 122.75) (width 0.2) (layer "F.Cu") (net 7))
 (segment (start 118.9 128.51) (end 113.14 122.75) (width 0.2) (layer "F.Cu") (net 7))
 (segment (start 135.67 103.42) (end 136.13 102.96) (width 0.2) (layer "F.Cu") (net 4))
 (segment (start 89.98 103.42) (end 135.67 103.42) (width 0.2) (layer "F.Cu") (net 4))
 (segment (start 89.96 106.42) (end 135.21 106.42) (width 0.2) (layer "F.Cu") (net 19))
 (segment (start 135.21 106.42) (end 136.13 105.5) (width 0.2) (layer "F.Cu") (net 19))
 (segment (start 89.98 97.39) (end 135.64 97.39) (width 0.2) (layer "F.Cu") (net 17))
 (segment (start 135.64 97.39) (end 136.13 97.88) (width 0.2) (layer "F.Cu") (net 17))
 (segment (start 89.98 100.42) (end 136.13 100.42) (width 0.2) (layer "F.Cu") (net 18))
 (segment (start 132.42 78.73) (end 136.13 75.02) (width 0.2) (layer "F.Cu") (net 8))
 (segment (start 99.63 78.73) (end 132.42 78.73) (width 0.2) (layer "F.Cu") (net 8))
 (segment (start 114.44 73.65) (end 136.13 95.34) (width 0.2) (layer "B.Cu") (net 16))
 (segment (start 99.63 73.65) (end 114.44 73.65) (width 0.2) (layer "B.Cu") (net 16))
 (segment (start 146.81 60.97) (end 137.43 70.35) (width 0.2) (layer "F.Cu") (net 11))
 (segment (start 137.43 81.74) (end 136.53 82.64) (width 0.2) (layer "F.Cu") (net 11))
 (segment (start 137.43 70.35) (end 137.43 81.74) (width 0.2) (layer "F.Cu") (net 11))
 (segment (start 136.53 82.64) (end 136.13 82.64) (width 0.2) (layer "F.Cu") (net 11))
 (segment (start 146.04 64.28) (end 146.04 75.27) (width 0.2) (layer "F.Cu") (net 12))
 (segment (start 146.04 75.27) (end 136.13 85.18) (width 0.2) (layer "F.Cu") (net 12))
 (segment (start 149.35 60.97) (end 146.04 64.28) (width 0.2) (layer "F.Cu") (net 12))
 (segment (start 99.63 71.11) (end 114.2 71.11) (width 0.2) (layer "B.Cu") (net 15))
 (segment (start 135.89 92.8) (end 136.13 92.8) (width 0.2) (layer "B.Cu") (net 15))
 (segment (start 114.2 71.11) (end 135.89 92.8) (width 0.2) (layer "B.Cu") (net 15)))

